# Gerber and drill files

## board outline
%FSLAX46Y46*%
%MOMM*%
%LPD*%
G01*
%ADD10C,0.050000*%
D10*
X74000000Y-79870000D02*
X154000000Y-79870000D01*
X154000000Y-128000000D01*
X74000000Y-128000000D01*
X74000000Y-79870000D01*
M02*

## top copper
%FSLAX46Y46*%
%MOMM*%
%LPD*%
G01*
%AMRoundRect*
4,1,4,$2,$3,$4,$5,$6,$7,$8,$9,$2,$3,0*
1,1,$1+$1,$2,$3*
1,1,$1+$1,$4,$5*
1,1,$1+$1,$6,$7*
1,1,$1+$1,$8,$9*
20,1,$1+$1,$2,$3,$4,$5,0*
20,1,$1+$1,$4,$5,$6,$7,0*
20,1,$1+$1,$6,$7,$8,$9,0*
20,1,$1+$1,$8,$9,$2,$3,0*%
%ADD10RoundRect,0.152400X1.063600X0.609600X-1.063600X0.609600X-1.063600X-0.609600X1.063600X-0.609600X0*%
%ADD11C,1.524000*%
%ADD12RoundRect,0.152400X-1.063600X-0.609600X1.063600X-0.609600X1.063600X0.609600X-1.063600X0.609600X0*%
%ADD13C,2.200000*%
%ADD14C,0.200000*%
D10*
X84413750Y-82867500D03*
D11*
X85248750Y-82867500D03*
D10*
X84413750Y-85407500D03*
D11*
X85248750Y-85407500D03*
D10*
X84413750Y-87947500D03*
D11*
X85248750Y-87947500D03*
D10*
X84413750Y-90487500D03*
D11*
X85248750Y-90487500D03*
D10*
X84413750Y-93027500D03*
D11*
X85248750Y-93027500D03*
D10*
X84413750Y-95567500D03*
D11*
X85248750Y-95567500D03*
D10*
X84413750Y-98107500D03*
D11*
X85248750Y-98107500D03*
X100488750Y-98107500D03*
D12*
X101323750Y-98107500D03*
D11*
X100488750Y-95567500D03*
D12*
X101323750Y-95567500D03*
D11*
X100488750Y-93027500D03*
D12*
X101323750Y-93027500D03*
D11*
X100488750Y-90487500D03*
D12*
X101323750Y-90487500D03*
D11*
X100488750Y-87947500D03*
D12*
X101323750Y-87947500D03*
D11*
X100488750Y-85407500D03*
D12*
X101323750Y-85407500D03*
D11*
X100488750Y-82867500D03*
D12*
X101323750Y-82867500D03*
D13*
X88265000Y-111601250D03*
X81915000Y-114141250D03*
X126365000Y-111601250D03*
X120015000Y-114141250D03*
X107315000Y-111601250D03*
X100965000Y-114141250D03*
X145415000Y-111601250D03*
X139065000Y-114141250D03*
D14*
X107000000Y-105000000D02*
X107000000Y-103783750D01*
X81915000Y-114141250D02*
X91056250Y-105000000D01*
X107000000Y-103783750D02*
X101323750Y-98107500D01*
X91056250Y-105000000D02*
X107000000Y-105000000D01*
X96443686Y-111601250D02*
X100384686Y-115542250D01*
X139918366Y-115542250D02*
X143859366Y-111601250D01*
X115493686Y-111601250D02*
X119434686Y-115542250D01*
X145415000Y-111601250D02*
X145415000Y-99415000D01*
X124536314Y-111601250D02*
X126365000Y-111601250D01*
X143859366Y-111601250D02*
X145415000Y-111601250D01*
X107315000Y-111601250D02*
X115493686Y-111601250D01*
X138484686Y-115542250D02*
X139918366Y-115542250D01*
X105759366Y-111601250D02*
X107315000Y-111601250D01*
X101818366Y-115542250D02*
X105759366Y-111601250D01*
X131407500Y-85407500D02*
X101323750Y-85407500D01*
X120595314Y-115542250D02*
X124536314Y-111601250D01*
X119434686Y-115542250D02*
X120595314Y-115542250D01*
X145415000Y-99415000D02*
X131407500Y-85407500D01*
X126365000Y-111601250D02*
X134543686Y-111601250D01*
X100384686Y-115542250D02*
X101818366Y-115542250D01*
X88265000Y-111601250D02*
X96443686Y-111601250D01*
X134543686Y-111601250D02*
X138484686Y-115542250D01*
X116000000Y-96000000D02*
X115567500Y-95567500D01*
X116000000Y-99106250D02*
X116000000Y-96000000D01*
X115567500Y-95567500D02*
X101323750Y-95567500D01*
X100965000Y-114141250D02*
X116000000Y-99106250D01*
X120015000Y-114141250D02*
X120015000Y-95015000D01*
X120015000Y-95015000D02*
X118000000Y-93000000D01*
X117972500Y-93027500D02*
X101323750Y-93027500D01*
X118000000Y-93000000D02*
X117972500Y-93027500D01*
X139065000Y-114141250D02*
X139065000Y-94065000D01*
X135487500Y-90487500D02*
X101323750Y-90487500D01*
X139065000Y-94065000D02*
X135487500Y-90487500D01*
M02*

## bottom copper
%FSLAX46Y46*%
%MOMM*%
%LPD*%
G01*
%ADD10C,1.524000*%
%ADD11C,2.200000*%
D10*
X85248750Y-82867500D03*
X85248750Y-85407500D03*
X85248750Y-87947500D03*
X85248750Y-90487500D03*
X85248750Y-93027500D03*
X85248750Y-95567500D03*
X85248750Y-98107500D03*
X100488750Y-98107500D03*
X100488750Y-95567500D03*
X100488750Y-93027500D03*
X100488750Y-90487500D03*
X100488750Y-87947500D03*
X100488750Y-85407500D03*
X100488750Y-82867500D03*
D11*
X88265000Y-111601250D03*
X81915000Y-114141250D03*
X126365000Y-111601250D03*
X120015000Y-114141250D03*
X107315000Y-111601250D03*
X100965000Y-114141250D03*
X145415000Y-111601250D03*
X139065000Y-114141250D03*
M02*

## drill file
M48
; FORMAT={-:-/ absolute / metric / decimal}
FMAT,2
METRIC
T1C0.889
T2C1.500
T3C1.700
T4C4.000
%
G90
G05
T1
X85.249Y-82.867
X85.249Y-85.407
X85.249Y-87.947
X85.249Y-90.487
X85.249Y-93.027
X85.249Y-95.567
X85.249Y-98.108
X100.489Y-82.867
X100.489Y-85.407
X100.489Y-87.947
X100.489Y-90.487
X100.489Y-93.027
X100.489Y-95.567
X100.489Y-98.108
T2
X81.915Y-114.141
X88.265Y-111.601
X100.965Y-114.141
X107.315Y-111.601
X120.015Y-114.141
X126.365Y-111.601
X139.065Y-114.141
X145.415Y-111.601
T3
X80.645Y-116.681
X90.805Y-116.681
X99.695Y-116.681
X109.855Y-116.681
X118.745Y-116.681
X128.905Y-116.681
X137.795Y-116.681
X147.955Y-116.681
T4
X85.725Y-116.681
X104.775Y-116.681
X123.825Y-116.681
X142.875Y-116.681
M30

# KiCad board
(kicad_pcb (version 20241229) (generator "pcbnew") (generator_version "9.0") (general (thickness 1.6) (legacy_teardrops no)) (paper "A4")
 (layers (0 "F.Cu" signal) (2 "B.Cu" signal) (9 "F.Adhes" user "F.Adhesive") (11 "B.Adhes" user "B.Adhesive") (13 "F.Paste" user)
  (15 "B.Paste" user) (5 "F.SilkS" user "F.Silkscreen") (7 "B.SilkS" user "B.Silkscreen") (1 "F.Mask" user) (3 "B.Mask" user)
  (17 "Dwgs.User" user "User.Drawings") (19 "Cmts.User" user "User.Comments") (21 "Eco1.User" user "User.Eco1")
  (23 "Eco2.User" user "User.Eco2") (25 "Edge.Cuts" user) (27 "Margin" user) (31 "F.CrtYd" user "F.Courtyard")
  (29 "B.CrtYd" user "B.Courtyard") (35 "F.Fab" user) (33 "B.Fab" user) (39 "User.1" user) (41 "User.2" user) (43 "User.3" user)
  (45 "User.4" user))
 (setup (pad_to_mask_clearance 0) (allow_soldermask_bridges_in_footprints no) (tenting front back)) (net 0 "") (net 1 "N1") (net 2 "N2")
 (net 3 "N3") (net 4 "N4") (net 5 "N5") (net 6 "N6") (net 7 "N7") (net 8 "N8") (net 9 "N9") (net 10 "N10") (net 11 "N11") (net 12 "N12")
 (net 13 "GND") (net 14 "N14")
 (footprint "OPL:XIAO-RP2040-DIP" (layer "F.Cu") (at 92.86875 90.4875)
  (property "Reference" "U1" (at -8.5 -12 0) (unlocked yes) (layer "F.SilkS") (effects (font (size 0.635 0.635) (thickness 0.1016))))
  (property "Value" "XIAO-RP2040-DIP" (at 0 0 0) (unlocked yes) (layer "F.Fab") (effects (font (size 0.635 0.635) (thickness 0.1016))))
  (pad "1" smd roundrect (at -8.455 -7.62 180) (size 2.432 1.524) (layers "F.Cu" "F.Mask") (roundrect_rratio 0.1) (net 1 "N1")
   (thermal_bridge_angle 45))
  (pad "1" thru_hole circle (at -7.62 -7.62 180) (size 1.524 1.524) (drill 0.889) (layers "*.Cu" "*.Mask") (remove_unused_layers no)
   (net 1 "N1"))
  (pad "2" smd roundrect (at -8.455 -5.08 180) (size 2.432 1.524) (layers "F.Cu" "F.Mask") (roundrect_rratio 0.1) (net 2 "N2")
   (thermal_bridge_angle 45))
  (pad "2" thru_hole circle (at -7.62 -5.08 180) (size 1.524 1.524) (drill 0.889) (layers "*.Cu" "*.Mask") (remove_unused_layers no)
   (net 2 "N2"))
  (pad "3" smd roundrect (at -8.455 -2.54 180) (size 2.432 1.524) (layers "F.Cu" "F.Mask") (roundrect_rratio 0.1) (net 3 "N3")
   (thermal_bridge_angle 45))
  (pad "3" thru_hole circle (at -7.62 -2.54 180) (size 1.524 1.524) (drill 0.889) (layers "*.Cu" "*.Mask") (remove_unused_layers no)
   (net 3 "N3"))
  (pad "4" smd roundrect (at -8.455 0 180) (size 2.432 1.524) (layers "F.Cu" "F.Mask") (roundrect_rratio 0.1) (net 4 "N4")
   (thermal_bridge_angle 45))
  (pad "4" thru_hole circle (at -7.62 0 180) (size 1.524 1.524) (drill 0.889) (layers "*.Cu" "*.Mask") (remove_unused_layers no)
   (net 4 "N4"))
  (pad "5" smd roundrect (at -8.455 2.54 180) (size 2.432 1.524) (layers "F.Cu" "F.Mask") (roundrect_rratio 0.1) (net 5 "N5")
   (thermal_bridge_angle 45))
  (pad "5" thru_hole circle (at -7.62 2.54 180) (size 1.524 1.524) (drill 0.889) (layers "*.Cu" "*.Mask") (remove_unused_layers no)
   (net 5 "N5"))
  (pad "6" smd roundrect (at -8.455 5.08 180) (size 2.432 1.524) (layers "F.Cu" "F.Mask") (roundrect_rratio 0.1) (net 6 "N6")
   (thermal_bridge_angle 45))
  (pad "6" thru_hole circle (at -7.62 5.08 180) (size 1.524 1.524) (drill 0.889) (layers "*.Cu" "*.Mask") (remove_unused_layers no)
   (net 6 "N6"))
  (pad "7" smd roundrect (at -8.455 7.62 180) (size 2.432 1.524) (layers "F.Cu" "F.Mask") (roundrect_rratio 0.1) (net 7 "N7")
   (thermal_bridge_angle 45))
  (pad "7" thru_hole circle (at -7.62 7.62 180) (size 1.524 1.524) (drill 0.889) (layers "*.Cu" "*.Mask") (remove_unused_layers no)
   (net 7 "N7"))
  (pad "8" thru_hole circle (at 7.62 7.62) (size 1.524 1.524) (drill 0.889) (layers "*.Cu" "*.Mask") (remove_unused_layers no) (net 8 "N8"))
  (pad "8" smd roundrect (at 8.455 7.62) (size 2.432 1.524) (layers "F.Cu" "F.Mask") (roundrect_rratio 0.1) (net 8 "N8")
   (thermal_bridge_angle 45))
  (pad "9" thru_hole circle (at 7.62 5.08) (size 1.524 1.524) (drill 0.889) (layers "*.Cu" "*.Mask") (remove_unused_layers no) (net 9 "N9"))
  (pad "9" smd roundrect (at 8.455 5.08) (size 2.432 1.524) (layers "F.Cu" "F.Mask") (roundrect_rratio 0.1) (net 9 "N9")
   (thermal_bridge_angle 45))
  (pad "10" thru_hole circle (at 7.62 2.54) (size 1.524 1.524) (drill 0.889) (layers "*.Cu" "*.Mask") (remove_unused_layers no)
   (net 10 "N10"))
  (pad "10" smd roundrect (at 8.455 2.54) (size 2.432 1.524) (layers "F.Cu" "F.Mask") (roundrect_rratio 0.1) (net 10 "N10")
   (thermal_bridge_angle 45))
  (pad "11" thru_hole circle (at 7.62 0) (size 1.524 1.524) (drill 0.889) (layers "*.Cu" "*.Mask") (remove_unused_layers no) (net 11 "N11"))
  (pad "11" smd roundrect (at 8.455 0) (size 2.432 1.524) (layers "F.Cu" "F.Mask") (roundrect_rratio 0.1) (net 11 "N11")
   (thermal_bridge_angle 45))
  (pad "12" thru_hole circle (at 7.62 -2.54) (size 1.524 1.524) (drill 0.889) (layers "*.Cu" "*.Mask") (remove_unused_layers no)
   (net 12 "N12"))
  (pad "12" smd roundrect (at 8.455 -2.54) (size 2.432 1.524) (layers "F.Cu" "F.Mask") (roundrect_rratio 0.1) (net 12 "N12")
   (thermal_bridge_angle 45))
  (pad "13" thru_hole circle (at 7.62 -5.08) (size 1.524 1.524) (drill 0.889) (layers "*.Cu" "*.Mask") (remove_unused_layers no)
   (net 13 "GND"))
  (pad "13" smd roundrect (at 8.455 -5.08) (size 2.432 1.524) (layers "F.Cu" "F.Mask") (roundrect_rratio 0.1) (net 13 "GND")
   (thermal_bridge_angle 45))
  (pad "14" thru_hole circle (at 7.62 -7.62) (size 1.524 1.524) (drill 0.889) (layers "*.Cu" "*.Mask") (remove_unused_layers no)
   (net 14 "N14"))
  (pad "14" smd roundrect (at 8.455 -7.62) (size 2.432 1.524) (layers "F.Cu" "F.Mask") (roundrect_rratio 0.1) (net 14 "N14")
   (thermal_bridge_angle 45)))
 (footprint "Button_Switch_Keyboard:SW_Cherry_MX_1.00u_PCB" (layer "F.Cu") (at 88.265 111.60125)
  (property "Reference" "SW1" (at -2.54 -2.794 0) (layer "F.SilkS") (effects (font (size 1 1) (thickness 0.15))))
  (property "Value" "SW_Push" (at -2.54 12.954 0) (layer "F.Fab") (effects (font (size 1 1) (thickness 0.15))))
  (pad "" np_thru_hole circle (at -7.62 5.08) (size 1.7 1.7) (drill 1.7) (layers "*.Cu" "*.Mask"))
  (pad "" np_thru_hole circle (at -2.54 5.08) (size 4 4) (drill 4) (layers "*.Cu" "*.Mask"))
  (pad "" np_thru_hole circle (at 2.54 5.08) (size 1.7 1.7) (drill 1.7) (layers "*.Cu" "*.Mask"))
  (pad "1" thru_hole circle (at 0 0) (size 2.2 2.2) (drill 1.5) (layers "*.Cu" "*.Mask") (remove_unused_layers no) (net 13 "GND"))
  (pad "2" thru_hole circle (at -6.35 2.54) (size 2.2 2.2) (drill 1.5) (layers "*.Cu" "*.Mask") (remove_unused_layers no) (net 8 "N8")))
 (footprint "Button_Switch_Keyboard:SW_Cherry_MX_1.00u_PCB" (layer "F.Cu") (at 126.365 111.60125)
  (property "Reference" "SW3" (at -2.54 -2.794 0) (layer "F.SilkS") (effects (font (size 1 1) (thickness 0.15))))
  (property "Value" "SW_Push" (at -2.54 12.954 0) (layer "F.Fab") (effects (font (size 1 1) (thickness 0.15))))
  (pad "" np_thru_hole circle (at -7.62 5.08) (size 1.7 1.7) (drill 1.7) (layers "*.Cu" "*.Mask"))
  (pad "" np_thru_hole circle (at -2.54 5.08) (size 4 4) (drill 4) (layers "*.Cu" "*.Mask"))
  (pad "" np_thru_hole circle (at 2.54 5.08) (size 1.7 1.7) (drill 1.7) (layers "*.Cu" "*.Mask"))
  (pad "1" thru_hole circle (at 0 0) (size 2.2 2.2) (drill 1.5) (layers "*.Cu" "*.Mask") (remove_unused_layers no) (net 13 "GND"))
  (pad "2" thru_hole circle (at -6.35 2.54) (size 2.2 2.2) (drill 1.5) (layers "*.Cu" "*.Mask") (remove_unused_layers no) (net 10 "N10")))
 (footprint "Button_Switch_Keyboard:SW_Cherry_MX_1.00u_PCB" (layer "F.Cu") (at 107.315 111.60125)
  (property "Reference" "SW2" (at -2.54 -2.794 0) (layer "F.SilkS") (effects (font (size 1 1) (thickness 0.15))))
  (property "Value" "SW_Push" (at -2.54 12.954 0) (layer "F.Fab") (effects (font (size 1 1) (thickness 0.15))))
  (pad "" np_thru_hole circle (at -7.62 5.08) (size 1.7 1.7) (drill 1.7) (layers "*.Cu" "*.Mask"))
  (pad "" np_thru_hole circle (at -2.54 5.08) (size 4 4) (drill 4) (layers "*.Cu" "*.Mask"))
  (pad "" np_thru_hole circle (at 2.54 5.08) (size 1.7 1.7) (drill 1.7) (layers "*.Cu" "*.Mask"))
  (pad "1" thru_hole circle (at 0 0) (size 2.2 2.2) (drill 1.5) (layers "*.Cu" "*.Mask") (remove_unused_layers no) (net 13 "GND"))
  (pad "2" thru_hole circle (at -6.35 2.54) (size 2.2 2.2) (drill 1.5) (layers "*.Cu" "*.Mask") (remove_unused_layers no) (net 9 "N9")))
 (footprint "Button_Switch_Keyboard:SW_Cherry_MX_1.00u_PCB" (layer "F.Cu") (at 145.415 111.60125)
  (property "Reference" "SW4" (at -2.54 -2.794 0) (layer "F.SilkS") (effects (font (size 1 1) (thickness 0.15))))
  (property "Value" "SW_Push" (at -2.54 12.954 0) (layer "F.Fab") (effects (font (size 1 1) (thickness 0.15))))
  (pad "" np_thru_hole circle (at -7.62 5.08) (size 1.7 1.7) (drill 1.7) (layers "*.Cu" "*.Mask"))
  (pad "" np_thru_hole circle (at -2.54 5.08) (size 4 4) (drill 4) (layers "*.Cu" "*.Mask"))
  (pad "" np_thru_hole circle (at 2.54 5.08) (size 1.7 1.7) (drill 1.7) (layers "*.Cu" "*.Mask"))
  (pad "1" thru_hole circle (at 0 0) (size 2.2 2.2) (drill 1.5) (layers "*.Cu" "*.Mask") (remove_unused_layers no) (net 13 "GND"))
  (pad "2" thru_hole circle (at -6.35 2.54) (size 2.2 2.2) (drill 1.5) (layers "*.Cu" "*.Mask") (remove_unused_layers no) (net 11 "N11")))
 (gr_rect (start 74 79.87) (end 154 128) (stroke (width 0.05) (type default)) (fill no) (layer "Edge.Cuts"))
 (segment (start 107 105) (end 107 103.78375) (width 0.2) (layer "F.Cu") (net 8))
 (segment (start 81.915 114.14125) (end 91.05625 105) (width 0.2) (layer "F.Cu") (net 8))
 (segment (start 107 103.78375) (end 101.32375 98.1075) (width 0.2) (layer "F.Cu") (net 8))
 (segment (start 91.05625 105) (end 107 105) (width 0.2) (layer "F.Cu") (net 8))
 (segment (start 96.443686 111.60125) (end 100.384686 115.54225) (width 0.2) (layer "F.Cu") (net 13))
 (segment (start 139.918366 115.54225) (end 143.859366 111.60125) (width 0.2) (layer "F.Cu") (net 13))
 (segment (start 115.493686 111.60125) (end 119.434686 115.54225) (width 0.2) (layer "F.Cu") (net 13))
 (segment (start 145.415 111.60125) (end 145.415 99.415) (width 0.2) (layer "F.Cu") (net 13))
 (segment (start 124.536314 111.60125) (end 126.365 111.60125) (width 0.2) (layer "F.Cu") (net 13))
 (segment (start 143.859366 111.60125) (end 145.415 111.60125) (width 0.2) (layer "F.Cu") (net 13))
 (segment (start 107.315 111.60125) (end 115.493686 111.60125) (width 0.2) (layer "F.Cu") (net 13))
 (segment (start 138.484686 115.54225) (end 139.918366 115.54225) (width 0.2) (layer "F.Cu") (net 13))
 (segment (start 105.759366 111.60125) (end 107.315 111.60125) (width 0.2) (layer "F.Cu") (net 13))
 (segment (start 101.818366 115.54225) (end 105.759366 111.60125) (width 0.2) (layer "F.Cu") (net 13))
 (segment (start 131.4075 85.4075) (end 101.32375 85.4075) (width 0.2) (layer "F.Cu") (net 13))
 (segment (start 120.595314 115.54225) (end 124.536314 111.60125) (width 0.2) (layer "F.Cu") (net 13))
 (segment (start 119.434686 115.54225) (end 120.595314 115.54225) (width 0.2) (layer "F.Cu") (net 13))
 (segment (start 145.415 99.415) (end 131.4075 85.4075) (width 0.2) (layer "F.Cu") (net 13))
 (segment (start 126.365 111.60125) (end 134.543686 111.60125) (width 0.2) (layer "F.Cu") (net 13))
 (segment (start 100.384686 115.54225) (end 101.818366 115.54225) (width 0.2) (layer "F.Cu") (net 13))
 (segment (start 88.265 111.60125) (end 96.443686 111.60125) (width 0.2) (layer "F.Cu") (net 13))
 (segment (start 134.543686 111.60125) (end 138.484686 115.54225) (width 0.2) (layer "F.Cu") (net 13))
 (segment (start 116 96) (end 115.5675 95.5675) (width 0.2) (layer "F.Cu") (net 9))
 (segment (start 116 99.10625) (end 116 96) (width 0.2) (layer "F.Cu") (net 9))
 (segment (start 115.5675 95.5675) (end 101.32375 95.5675) (width 0.2) (layer "F.Cu") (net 9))
 (segment (start 100.965 114.14125) (end 116 99.10625) (width 0.2) (layer "F.Cu") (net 9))
 (segment (start 120.015 114.14125) (end 120.015 95.015) (width 0.2) (layer "F.Cu") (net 10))
 (segment (start 120.015 95.015) (end 118 93) (width 0.2) (layer "F.Cu") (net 10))
 (segment (start 117.9725 93.0275) (end 101.32375 93.0275) (width 0.2) (layer "F.Cu") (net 10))
 (segment (start 118 93) (end 117.9725 93.0275) (width 0.2) (layer "F.Cu") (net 10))
 (segment (start 139.065 114.14125) (end 139.065 94.065) (width 0.2) (layer "F.Cu") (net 11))
 (segment (start 135.4875 90.4875) (end 101.32375 90.4875) (width 0.2) (layer "F.Cu") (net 11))
 (segment (start 139.065 94.065) (end 135.4875 90.4875) (width 0.2) (layer "F.Cu") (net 11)))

